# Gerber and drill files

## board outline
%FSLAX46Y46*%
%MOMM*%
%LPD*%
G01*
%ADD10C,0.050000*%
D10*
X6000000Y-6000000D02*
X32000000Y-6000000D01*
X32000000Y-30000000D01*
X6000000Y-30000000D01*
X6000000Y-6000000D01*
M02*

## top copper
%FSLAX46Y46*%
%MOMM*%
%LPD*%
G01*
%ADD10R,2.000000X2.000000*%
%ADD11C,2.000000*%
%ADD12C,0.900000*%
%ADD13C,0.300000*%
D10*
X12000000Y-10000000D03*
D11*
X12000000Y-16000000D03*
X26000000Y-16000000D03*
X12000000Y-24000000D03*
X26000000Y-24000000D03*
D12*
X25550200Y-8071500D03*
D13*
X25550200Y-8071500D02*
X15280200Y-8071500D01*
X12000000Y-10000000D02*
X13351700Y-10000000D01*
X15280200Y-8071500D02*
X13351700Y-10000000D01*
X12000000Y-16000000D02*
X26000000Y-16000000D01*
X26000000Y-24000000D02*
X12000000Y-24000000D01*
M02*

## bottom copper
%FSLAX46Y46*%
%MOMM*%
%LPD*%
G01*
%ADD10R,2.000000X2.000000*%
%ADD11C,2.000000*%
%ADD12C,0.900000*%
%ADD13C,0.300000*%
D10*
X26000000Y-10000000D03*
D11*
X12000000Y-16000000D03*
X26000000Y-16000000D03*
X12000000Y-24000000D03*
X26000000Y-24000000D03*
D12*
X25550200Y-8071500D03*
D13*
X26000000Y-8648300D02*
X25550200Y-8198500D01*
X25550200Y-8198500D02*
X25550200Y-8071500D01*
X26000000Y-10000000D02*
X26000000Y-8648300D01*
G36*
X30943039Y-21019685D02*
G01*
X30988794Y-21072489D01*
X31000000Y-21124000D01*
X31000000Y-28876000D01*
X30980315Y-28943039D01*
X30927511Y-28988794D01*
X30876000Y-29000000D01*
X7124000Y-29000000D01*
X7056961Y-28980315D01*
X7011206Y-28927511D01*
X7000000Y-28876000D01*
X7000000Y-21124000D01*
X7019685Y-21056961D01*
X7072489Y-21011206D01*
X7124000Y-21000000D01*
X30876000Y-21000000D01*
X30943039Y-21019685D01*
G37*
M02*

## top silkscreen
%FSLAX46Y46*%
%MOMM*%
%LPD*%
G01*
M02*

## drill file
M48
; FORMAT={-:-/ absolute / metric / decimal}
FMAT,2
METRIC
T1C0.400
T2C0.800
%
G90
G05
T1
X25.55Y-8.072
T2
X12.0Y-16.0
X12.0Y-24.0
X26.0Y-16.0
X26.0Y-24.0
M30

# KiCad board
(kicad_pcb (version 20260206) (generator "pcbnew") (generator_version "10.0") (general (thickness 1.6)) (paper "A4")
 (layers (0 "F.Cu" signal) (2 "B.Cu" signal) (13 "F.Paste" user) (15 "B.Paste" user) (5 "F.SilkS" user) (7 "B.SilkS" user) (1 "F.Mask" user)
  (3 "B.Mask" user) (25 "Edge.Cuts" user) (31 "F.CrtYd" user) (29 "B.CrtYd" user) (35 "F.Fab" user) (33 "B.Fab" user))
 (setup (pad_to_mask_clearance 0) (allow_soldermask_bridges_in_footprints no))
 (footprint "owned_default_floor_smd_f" (layer "F.Cu") (at 12 10)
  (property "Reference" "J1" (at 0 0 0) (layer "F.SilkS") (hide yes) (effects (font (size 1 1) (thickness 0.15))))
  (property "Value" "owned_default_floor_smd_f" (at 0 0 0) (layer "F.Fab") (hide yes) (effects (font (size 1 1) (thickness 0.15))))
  (pad "1" smd rect (at 0 0) (size 2 2) (layers "F.Cu" "F.Paste" "F.Mask") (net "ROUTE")))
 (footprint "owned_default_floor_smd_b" (layer "B.Cu") (at 26 10)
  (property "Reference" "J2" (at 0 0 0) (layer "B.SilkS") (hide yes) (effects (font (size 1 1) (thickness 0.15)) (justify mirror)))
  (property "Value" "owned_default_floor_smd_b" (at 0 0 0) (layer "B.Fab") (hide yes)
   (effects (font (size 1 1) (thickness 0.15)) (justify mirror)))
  (pad "1" smd rect (at 0 0) (size 2 2) (layers "B.Cu" "B.Paste" "B.Mask") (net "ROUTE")))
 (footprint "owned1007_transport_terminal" (layer "F.Cu") (at 12 16)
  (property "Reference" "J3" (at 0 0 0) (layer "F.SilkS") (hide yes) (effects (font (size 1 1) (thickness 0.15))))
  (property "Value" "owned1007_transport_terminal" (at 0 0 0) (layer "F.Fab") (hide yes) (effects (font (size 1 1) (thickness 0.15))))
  (pad "1" thru_hole circle (at 0 0) (size 2 2) (drill 0.8) (layers "*.Cu" "*.Mask") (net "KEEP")))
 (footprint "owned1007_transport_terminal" (layer "F.Cu") (at 26 16)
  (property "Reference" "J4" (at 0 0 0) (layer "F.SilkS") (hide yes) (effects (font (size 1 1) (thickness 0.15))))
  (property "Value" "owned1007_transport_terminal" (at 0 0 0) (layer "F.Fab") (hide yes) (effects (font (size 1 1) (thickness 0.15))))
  (pad "1" thru_hole circle (at 0 0) (size 2 2) (drill 0.8) (layers "*.Cu" "*.Mask") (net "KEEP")))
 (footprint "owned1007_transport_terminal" (layer "F.Cu") (at 12 24)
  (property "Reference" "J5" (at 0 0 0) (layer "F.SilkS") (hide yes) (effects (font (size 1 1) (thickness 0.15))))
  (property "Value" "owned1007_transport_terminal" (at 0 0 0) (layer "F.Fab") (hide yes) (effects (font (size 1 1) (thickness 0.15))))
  (pad "1" thru_hole circle (at 0 0) (size 2 2) (drill 0.8) (layers "*.Cu" "*.Mask") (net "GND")))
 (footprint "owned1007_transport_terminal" (layer "F.Cu") (at 26 24)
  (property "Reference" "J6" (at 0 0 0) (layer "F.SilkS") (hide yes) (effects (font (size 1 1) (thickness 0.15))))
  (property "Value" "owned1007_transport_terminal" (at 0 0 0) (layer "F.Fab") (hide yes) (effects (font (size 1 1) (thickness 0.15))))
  (pad "1" thru_hole circle (at 0 0) (size 2 2) (drill 0.8) (layers "*.Cu" "*.Mask") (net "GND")))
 (gr_rect (start 6 6) (end 32 30) (stroke (width 0.05) (type default)) (fill none) (layer "Edge.Cuts"))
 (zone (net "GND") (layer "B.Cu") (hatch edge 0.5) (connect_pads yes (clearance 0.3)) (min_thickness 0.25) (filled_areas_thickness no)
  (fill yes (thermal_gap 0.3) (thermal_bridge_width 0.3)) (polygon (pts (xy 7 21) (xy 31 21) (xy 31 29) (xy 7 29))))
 (segment (start 25.5502 8.0715) (end 15.2802 8.0715) (width 0.3) (layer "F.Cu") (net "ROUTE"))
 (segment (start 12 10) (end 13.3517 10) (width 0.3) (layer "F.Cu") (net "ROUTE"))
 (segment (start 15.2802 8.0715) (end 13.3517 10) (width 0.3) (layer "F.Cu") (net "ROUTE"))
 (via (at 25.5502 8.0715) (size 0.9) (drill 0.4) (layers "F.Cu" "B.Cu") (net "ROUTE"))
 (segment (start 26 8.6483) (end 25.5502 8.1985) (width 0.3) (layer "B.Cu") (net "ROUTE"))
 (segment (start 25.5502 8.1985) (end 25.5502 8.0715) (width 0.3) (layer "B.Cu") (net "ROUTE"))
 (segment (start 26 10) (end 26 8.6483) (width 0.3) (layer "B.Cu") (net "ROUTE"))
 (segment (start 12 16) (end 26 16) (width 0.3) (layer "F.Cu") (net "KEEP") (locked yes))
 (segment (start 26 24) (end 12 24) (width 0.3) (layer "F.Cu") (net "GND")))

